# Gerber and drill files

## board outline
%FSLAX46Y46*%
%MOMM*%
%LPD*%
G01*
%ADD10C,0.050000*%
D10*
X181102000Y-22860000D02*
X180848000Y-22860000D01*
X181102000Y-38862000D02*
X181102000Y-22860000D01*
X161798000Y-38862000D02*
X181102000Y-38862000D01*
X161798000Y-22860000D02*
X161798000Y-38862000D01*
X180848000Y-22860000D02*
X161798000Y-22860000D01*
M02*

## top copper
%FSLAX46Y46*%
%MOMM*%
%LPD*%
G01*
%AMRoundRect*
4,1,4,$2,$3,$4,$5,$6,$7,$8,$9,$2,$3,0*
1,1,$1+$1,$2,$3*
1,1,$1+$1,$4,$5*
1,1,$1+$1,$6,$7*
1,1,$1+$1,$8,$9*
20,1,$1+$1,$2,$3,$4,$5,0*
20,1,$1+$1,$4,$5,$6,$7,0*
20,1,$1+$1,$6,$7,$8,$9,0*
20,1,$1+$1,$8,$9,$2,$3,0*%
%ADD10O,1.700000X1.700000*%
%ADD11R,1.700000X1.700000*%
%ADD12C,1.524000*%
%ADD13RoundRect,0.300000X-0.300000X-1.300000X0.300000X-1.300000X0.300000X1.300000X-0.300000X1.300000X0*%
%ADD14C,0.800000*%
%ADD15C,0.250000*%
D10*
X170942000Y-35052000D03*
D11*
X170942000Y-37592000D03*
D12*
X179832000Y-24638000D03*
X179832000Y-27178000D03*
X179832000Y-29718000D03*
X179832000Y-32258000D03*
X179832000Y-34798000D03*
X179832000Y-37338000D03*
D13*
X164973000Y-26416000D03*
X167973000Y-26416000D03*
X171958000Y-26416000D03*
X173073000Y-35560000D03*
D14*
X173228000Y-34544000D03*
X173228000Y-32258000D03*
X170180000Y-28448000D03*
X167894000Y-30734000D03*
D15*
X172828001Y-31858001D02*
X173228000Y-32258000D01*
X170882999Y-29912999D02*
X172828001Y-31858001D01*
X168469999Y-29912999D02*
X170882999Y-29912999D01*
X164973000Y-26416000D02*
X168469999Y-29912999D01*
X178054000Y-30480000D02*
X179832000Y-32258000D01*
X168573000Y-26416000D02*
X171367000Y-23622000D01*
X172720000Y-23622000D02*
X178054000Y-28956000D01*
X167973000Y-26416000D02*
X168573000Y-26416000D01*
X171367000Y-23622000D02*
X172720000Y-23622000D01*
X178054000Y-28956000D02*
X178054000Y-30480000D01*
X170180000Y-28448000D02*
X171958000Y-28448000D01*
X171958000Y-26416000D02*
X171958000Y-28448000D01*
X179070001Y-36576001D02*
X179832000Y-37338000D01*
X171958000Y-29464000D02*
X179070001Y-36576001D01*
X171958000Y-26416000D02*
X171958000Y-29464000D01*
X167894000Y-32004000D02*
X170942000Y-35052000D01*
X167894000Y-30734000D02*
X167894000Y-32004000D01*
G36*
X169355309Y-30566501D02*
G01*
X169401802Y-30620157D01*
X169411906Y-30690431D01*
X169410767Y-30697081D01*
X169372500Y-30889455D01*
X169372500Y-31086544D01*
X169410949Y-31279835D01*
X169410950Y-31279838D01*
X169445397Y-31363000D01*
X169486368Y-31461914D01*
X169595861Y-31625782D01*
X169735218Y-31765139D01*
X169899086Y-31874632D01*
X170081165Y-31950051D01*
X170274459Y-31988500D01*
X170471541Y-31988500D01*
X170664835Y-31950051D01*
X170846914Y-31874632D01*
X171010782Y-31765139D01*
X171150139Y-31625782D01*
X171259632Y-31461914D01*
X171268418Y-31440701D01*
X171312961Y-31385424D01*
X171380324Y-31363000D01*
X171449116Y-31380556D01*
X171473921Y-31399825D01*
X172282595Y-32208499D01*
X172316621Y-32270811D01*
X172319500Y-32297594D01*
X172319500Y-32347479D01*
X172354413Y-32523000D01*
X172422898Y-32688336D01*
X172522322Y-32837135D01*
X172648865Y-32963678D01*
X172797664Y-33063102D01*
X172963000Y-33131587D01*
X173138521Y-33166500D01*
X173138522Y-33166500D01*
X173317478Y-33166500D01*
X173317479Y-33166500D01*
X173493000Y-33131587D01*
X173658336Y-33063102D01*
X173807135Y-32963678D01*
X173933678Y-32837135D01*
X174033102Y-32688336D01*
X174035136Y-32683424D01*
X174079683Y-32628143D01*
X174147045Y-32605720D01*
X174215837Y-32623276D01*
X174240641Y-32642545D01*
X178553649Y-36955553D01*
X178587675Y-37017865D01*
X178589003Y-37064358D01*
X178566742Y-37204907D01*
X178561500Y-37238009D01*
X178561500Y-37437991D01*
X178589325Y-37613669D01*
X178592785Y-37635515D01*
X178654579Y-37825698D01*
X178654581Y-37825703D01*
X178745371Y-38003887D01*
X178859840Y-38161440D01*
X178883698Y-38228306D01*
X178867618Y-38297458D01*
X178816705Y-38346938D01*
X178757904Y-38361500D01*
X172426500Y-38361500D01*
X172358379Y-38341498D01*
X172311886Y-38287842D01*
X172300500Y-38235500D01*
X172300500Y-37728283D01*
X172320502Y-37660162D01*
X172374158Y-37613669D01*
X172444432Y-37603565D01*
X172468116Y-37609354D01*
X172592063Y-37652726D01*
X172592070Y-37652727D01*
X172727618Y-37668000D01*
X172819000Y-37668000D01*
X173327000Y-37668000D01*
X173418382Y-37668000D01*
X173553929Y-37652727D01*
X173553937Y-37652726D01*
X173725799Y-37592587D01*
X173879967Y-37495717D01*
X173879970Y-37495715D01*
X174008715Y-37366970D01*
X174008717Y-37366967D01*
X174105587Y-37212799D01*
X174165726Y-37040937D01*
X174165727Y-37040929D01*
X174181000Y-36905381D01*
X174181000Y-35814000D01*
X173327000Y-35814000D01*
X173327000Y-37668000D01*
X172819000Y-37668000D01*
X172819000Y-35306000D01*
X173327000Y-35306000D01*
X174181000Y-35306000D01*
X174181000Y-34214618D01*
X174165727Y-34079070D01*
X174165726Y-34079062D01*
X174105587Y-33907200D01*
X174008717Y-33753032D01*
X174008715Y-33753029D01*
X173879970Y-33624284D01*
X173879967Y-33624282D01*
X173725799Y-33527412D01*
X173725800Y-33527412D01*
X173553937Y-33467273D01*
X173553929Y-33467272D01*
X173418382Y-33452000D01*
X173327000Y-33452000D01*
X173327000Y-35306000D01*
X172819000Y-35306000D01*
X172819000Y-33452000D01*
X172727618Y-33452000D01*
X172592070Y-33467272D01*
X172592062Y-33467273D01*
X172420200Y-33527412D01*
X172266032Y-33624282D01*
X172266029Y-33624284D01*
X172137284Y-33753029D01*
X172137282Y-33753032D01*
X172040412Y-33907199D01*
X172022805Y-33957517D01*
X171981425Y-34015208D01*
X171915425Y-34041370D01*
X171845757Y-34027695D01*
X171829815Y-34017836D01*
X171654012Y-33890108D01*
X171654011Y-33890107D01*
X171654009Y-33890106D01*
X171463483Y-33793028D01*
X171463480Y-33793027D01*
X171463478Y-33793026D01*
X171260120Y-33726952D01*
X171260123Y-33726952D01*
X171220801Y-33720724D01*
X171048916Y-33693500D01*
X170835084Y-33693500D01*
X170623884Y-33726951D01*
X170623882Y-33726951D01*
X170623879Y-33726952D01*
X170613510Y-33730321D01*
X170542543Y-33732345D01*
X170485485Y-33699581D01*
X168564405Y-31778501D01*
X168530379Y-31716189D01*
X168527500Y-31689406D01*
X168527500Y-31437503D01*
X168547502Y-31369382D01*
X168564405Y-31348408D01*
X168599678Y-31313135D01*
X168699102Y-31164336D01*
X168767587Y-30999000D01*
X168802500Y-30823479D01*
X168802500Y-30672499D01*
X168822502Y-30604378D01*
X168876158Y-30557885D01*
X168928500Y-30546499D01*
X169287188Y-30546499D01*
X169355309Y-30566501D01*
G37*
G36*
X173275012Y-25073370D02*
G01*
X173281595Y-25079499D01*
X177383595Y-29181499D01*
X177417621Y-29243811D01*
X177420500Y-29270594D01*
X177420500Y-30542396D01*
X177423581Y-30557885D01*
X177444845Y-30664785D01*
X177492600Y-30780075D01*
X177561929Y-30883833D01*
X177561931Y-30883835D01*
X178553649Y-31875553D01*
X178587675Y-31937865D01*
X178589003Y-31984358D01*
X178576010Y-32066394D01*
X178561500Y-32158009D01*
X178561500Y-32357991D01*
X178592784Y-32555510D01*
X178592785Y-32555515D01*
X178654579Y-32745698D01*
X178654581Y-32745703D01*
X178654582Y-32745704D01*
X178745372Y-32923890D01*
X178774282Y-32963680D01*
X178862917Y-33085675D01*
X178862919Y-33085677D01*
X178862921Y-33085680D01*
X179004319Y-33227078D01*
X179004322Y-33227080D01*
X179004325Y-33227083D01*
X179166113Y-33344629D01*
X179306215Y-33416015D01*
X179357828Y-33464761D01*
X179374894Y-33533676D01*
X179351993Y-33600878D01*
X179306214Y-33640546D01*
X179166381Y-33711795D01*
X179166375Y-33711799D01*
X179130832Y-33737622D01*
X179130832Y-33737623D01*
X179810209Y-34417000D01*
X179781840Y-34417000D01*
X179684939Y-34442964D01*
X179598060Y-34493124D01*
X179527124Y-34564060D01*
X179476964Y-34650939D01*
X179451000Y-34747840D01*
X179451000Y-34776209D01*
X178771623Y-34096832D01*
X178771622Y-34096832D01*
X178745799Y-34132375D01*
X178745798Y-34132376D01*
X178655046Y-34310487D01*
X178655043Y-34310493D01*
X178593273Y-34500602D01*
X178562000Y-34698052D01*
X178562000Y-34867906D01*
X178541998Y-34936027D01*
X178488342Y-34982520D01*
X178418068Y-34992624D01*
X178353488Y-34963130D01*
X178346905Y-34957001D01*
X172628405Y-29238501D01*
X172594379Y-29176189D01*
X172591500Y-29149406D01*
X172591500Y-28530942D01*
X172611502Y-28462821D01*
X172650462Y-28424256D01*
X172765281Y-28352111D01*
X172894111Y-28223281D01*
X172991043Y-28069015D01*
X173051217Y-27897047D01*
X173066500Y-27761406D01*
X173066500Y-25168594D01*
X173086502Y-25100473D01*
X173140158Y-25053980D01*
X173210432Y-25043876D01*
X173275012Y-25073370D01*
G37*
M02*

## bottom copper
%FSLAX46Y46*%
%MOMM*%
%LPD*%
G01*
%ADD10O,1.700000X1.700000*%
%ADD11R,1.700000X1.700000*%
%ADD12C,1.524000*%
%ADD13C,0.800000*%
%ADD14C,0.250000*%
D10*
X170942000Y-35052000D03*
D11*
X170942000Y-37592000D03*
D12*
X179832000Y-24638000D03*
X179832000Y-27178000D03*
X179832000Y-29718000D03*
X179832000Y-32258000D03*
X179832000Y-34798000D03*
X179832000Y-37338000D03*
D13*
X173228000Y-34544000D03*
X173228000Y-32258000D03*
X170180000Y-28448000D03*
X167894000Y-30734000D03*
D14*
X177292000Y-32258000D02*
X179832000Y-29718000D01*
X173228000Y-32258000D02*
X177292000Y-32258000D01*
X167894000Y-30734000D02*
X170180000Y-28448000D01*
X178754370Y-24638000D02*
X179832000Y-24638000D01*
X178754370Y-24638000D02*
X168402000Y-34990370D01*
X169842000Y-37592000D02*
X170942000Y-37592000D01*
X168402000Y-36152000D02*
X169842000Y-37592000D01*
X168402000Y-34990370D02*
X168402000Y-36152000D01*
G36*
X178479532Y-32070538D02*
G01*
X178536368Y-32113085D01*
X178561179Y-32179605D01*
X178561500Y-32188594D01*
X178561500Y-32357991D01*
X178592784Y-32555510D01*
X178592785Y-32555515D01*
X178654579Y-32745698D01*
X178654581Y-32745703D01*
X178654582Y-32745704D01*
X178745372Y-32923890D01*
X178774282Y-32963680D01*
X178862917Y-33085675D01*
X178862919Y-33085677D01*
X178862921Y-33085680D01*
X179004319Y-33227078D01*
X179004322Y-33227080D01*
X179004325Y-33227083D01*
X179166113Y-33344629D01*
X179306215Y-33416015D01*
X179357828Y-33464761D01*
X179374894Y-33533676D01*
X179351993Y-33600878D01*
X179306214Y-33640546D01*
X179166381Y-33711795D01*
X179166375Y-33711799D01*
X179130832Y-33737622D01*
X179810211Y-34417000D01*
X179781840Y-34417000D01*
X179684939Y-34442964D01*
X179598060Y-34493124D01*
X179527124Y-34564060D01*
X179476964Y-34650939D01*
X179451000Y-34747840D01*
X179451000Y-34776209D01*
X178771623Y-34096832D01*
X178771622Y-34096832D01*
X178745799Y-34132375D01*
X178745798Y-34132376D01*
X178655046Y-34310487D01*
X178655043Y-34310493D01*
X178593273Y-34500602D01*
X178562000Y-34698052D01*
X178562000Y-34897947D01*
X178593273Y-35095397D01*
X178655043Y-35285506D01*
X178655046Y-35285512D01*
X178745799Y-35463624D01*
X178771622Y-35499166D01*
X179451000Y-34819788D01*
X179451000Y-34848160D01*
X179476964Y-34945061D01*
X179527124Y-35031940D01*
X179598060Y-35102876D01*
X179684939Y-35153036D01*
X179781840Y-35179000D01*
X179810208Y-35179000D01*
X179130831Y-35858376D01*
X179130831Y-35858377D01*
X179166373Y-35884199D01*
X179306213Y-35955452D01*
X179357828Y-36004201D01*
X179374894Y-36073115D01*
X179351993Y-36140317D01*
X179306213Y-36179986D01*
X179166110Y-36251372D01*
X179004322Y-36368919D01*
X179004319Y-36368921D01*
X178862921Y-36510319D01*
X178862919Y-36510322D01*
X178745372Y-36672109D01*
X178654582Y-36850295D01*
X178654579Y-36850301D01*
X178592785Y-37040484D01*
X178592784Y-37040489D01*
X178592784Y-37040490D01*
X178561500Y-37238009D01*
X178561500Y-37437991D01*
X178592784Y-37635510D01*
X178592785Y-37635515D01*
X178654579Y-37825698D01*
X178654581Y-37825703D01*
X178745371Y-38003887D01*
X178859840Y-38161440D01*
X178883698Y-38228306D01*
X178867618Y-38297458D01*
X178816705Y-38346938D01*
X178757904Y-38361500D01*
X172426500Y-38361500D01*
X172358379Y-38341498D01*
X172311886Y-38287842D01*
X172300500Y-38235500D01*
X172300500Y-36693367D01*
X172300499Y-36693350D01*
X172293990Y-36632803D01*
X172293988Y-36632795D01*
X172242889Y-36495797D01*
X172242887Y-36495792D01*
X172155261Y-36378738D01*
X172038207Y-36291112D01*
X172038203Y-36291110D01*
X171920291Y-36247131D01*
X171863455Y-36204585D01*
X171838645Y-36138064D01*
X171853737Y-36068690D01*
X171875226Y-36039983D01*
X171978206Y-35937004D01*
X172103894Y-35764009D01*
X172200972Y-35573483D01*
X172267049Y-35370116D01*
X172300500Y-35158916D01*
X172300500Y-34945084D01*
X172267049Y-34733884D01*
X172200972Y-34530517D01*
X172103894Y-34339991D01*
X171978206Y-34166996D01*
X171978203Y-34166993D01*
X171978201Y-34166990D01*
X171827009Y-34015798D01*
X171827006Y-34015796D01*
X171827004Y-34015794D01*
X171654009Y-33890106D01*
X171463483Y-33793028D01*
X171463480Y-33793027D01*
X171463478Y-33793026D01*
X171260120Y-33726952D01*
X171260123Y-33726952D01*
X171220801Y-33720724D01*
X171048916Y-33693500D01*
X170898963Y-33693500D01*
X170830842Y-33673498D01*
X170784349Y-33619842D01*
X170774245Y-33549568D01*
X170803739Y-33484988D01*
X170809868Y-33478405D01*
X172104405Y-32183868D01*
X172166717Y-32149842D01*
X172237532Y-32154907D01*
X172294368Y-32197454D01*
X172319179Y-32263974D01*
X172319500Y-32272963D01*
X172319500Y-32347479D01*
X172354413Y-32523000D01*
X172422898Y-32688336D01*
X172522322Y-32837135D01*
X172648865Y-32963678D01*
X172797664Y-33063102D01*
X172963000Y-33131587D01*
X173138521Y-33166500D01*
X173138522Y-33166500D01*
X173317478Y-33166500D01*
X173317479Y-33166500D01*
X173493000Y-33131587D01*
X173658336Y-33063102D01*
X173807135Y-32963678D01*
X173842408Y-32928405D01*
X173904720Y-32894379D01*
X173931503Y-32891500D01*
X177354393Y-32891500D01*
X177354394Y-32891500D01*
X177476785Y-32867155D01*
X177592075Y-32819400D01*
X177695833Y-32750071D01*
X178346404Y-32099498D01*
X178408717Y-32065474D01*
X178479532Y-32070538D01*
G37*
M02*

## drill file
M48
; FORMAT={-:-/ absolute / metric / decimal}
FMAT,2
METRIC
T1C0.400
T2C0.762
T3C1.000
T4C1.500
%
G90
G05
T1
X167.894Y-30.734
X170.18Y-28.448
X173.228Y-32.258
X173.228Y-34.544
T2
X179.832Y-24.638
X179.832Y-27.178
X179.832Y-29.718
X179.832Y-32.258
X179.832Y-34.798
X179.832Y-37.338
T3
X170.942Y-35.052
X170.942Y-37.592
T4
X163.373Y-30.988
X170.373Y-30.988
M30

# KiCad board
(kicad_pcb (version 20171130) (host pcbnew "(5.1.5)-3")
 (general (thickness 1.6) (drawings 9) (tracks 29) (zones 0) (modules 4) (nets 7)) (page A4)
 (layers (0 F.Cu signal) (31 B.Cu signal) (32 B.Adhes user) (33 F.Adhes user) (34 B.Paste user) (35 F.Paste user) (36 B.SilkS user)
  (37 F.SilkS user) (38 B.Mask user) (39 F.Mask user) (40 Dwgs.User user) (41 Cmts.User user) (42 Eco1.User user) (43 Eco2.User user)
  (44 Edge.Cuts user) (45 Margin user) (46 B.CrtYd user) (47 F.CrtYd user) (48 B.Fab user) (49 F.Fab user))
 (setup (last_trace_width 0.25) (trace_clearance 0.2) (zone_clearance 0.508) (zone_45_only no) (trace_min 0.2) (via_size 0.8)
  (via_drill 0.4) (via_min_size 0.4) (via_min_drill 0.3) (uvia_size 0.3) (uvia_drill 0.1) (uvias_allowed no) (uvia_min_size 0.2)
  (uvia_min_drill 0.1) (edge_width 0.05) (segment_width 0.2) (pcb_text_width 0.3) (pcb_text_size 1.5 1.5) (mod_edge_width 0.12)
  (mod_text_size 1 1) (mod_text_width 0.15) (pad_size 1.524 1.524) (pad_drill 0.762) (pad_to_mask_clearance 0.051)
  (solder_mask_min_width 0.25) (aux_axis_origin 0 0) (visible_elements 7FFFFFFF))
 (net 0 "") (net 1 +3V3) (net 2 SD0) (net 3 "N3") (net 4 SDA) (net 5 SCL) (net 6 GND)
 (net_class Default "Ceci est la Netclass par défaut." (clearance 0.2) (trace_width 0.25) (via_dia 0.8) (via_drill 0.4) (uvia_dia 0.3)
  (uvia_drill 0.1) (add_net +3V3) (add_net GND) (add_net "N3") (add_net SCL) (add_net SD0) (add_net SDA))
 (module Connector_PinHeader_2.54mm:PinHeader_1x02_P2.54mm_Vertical (layer F.Cu) (at 170.942 37.592 180)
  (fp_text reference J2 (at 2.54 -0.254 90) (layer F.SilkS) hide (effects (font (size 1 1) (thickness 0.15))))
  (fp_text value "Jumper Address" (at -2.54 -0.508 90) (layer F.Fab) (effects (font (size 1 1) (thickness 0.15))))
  (pad 2 thru_hole oval (at 0 2.54 180) (size 1.7 1.7) (drill 1) (layers *.Cu *.Mask) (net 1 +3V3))
  (pad 1 thru_hole rect (at 0 0 180) (size 1.7 1.7) (drill 1) (layers *.Cu *.Mask) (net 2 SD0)))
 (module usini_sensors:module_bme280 (layer F.Cu) (at 174.752 24.892 180)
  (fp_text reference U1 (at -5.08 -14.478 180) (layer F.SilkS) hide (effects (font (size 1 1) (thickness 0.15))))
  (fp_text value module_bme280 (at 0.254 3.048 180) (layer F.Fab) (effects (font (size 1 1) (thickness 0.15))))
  (pad 6 thru_hole circle (at -5.08 0.254 180) (size 1.524 1.524) (drill 0.762) (layers *.Cu *.Mask) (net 2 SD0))
  (pad 5 thru_hole circle (at -5.08 -2.286 180) (size 1.524 1.524) (drill 0.762) (layers *.Cu *.Mask) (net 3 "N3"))
  (pad 4 thru_hole circle (at -5.08 -4.826 180) (size 1.524 1.524) (drill 0.762) (layers *.Cu *.Mask) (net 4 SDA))
  (pad 3 thru_hole circle (at -5.08 -7.366 180) (size 1.524 1.524) (drill 0.762) (layers *.Cu *.Mask) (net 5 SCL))
  (pad 2 thru_hole circle (at -5.08 -9.906 180) (size 1.524 1.524) (drill 0.762) (layers *.Cu *.Mask) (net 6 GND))
  (pad 1 thru_hole circle (at -5.08 -12.446 180) (size 1.524 1.524) (drill 0.762) (layers *.Cu *.Mask) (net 1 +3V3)))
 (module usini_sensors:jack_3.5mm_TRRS (layer F.Cu) (at 168.148 30.988)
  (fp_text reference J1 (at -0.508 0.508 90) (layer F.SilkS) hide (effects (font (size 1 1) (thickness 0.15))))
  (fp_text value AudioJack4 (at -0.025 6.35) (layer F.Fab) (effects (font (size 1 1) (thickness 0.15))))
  (pad "" np_thru_hole circle (at 2.225 0) (size 1.5 1.5) (drill 1.5) (layers *.Cu *.Mask))
  (pad "" np_thru_hole circle (at -4.775 0) (size 1.5 1.5) (drill 1.5) (layers *.Cu *.Mask))
  (pad R2 smd roundrect (at -3.175 -4.572) (size 1.2 3.2) (layers F.Cu F.Paste F.Mask) (roundrect_rratio 0.25) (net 4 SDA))
  (pad R1 smd roundrect (at -0.175 -4.572) (size 1.2 3.2) (layers F.Cu F.Paste F.Mask) (roundrect_rratio 0.25) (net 5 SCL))
  (pad T smd roundrect (at 3.81 -4.572) (size 1.2 3.2) (layers F.Cu F.Paste F.Mask) (roundrect_rratio 0.25) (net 1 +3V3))
  (pad S smd roundrect (at 4.925 4.572) (size 1.2 3.2) (layers F.Cu F.Paste F.Mask) (roundrect_rratio 0.25) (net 6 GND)))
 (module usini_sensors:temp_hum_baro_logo (layer B.Cu) (at 173.736 27.686 180)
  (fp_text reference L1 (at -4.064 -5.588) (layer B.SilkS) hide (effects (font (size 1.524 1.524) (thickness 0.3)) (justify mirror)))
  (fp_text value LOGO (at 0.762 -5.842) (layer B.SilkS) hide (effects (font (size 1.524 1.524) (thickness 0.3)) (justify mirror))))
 (gr_line (start 181.102 22.86) (end 180.848 22.86) (layer Edge.Cuts) (width 0.05))
 (gr_line (start 181.102 38.862) (end 181.102 22.86) (layer Edge.Cuts) (width 0.05))
 (gr_line (start 161.798 38.862) (end 181.102 38.862) (layer Edge.Cuts) (width 0.05))
 (gr_line (start 161.798 22.86) (end 161.798 38.862) (layer Edge.Cuts) (width 0.05))
 (gr_line (start 180.848 22.86) (end 161.798 22.86) (layer Edge.Cuts) (width 0.05))
 (via (at 173.228 34.544) (size 0.8) (drill 0.4) (layers F.Cu B.Cu) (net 6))
 (via (at 173.228 32.258) (size 0.8) (drill 0.4) (layers F.Cu B.Cu) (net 4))
 (segment (start 177.292 32.258) (end 179.832 29.718) (width 0.25) (layer B.Cu) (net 4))
 (segment (start 173.228 32.258) (end 177.292 32.258) (width 0.25) (layer B.Cu) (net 4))
 (segment (start 172.828001 31.858001) (end 173.228 32.258) (width 0.25) (layer F.Cu) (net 4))
 (segment (start 170.882999 29.912999) (end 172.828001 31.858001) (width 0.25) (layer F.Cu) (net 4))
 (segment (start 168.469999 29.912999) (end 170.882999 29.912999) (width 0.25) (layer F.Cu) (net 4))
 (segment (start 164.973 26.416) (end 168.469999 29.912999) (width 0.25) (layer F.Cu) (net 4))
 (segment (start 178.054 30.48) (end 179.832 32.258) (width 0.25) (layer F.Cu) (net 5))
 (segment (start 168.573 26.416) (end 171.367 23.622) (width 0.25) (layer F.Cu) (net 5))
 (segment (start 172.72 23.622) (end 178.054 28.956) (width 0.25) (layer F.Cu) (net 5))
 (segment (start 167.973 26.416) (end 168.573 26.416) (width 0.25) (layer F.Cu) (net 5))
 (segment (start 171.367 23.622) (end 172.72 23.622) (width 0.25) (layer F.Cu) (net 5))
 (segment (start 178.054 28.956) (end 178.054 30.48) (width 0.25) (layer F.Cu) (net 5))
 (via (at 170.18 28.448) (size 0.8) (drill 0.4) (layers F.Cu B.Cu) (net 1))
 (segment (start 170.18 28.448) (end 171.958 28.448) (width 0.25) (layer F.Cu) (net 1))
 (segment (start 171.958 26.416) (end 171.958 28.448) (width 0.25) (layer F.Cu) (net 1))
 (segment (start 179.070001 36.576001) (end 179.832 37.338) (width 0.25) (layer F.Cu) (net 1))
 (segment (start 171.958 29.464) (end 179.070001 36.576001) (width 0.25) (layer F.Cu) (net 1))
 (segment (start 171.958 26.416) (end 171.958 29.464) (width 0.25) (layer F.Cu) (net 1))
 (via (at 167.894 30.734) (size 0.8) (drill 0.4) (layers F.Cu B.Cu) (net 1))
 (segment (start 167.894 30.734) (end 170.18 28.448) (width 0.25) (layer B.Cu) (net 1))
 (segment (start 167.894 32.004) (end 170.942 35.052) (width 0.25) (layer F.Cu) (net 1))
 (segment (start 167.894 30.734) (end 167.894 32.004) (width 0.25) (layer F.Cu) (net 1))
 (segment (start 178.75437 24.638) (end 179.832 24.638) (width 0.25) (layer B.Cu) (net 2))
 (segment (start 178.75437 24.638) (end 168.402 34.99037) (width 0.25) (layer B.Cu) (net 2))
 (segment (start 169.842 37.592) (end 170.942 37.592) (width 0.25) (layer B.Cu) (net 2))
 (segment (start 168.402 36.152) (end 169.842 37.592) (width 0.25) (layer B.Cu) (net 2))
 (segment (start 168.402 34.99037) (end 168.402 36.152) (width 0.25) (layer B.Cu) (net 2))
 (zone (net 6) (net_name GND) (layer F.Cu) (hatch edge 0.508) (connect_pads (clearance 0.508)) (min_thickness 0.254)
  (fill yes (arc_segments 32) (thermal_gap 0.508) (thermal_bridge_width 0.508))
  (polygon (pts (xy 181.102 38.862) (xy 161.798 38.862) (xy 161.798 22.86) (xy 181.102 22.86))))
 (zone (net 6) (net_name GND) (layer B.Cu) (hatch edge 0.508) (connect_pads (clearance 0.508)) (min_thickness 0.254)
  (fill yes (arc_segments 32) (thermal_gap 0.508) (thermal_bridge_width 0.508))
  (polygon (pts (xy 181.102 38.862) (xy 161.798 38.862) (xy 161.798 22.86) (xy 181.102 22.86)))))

